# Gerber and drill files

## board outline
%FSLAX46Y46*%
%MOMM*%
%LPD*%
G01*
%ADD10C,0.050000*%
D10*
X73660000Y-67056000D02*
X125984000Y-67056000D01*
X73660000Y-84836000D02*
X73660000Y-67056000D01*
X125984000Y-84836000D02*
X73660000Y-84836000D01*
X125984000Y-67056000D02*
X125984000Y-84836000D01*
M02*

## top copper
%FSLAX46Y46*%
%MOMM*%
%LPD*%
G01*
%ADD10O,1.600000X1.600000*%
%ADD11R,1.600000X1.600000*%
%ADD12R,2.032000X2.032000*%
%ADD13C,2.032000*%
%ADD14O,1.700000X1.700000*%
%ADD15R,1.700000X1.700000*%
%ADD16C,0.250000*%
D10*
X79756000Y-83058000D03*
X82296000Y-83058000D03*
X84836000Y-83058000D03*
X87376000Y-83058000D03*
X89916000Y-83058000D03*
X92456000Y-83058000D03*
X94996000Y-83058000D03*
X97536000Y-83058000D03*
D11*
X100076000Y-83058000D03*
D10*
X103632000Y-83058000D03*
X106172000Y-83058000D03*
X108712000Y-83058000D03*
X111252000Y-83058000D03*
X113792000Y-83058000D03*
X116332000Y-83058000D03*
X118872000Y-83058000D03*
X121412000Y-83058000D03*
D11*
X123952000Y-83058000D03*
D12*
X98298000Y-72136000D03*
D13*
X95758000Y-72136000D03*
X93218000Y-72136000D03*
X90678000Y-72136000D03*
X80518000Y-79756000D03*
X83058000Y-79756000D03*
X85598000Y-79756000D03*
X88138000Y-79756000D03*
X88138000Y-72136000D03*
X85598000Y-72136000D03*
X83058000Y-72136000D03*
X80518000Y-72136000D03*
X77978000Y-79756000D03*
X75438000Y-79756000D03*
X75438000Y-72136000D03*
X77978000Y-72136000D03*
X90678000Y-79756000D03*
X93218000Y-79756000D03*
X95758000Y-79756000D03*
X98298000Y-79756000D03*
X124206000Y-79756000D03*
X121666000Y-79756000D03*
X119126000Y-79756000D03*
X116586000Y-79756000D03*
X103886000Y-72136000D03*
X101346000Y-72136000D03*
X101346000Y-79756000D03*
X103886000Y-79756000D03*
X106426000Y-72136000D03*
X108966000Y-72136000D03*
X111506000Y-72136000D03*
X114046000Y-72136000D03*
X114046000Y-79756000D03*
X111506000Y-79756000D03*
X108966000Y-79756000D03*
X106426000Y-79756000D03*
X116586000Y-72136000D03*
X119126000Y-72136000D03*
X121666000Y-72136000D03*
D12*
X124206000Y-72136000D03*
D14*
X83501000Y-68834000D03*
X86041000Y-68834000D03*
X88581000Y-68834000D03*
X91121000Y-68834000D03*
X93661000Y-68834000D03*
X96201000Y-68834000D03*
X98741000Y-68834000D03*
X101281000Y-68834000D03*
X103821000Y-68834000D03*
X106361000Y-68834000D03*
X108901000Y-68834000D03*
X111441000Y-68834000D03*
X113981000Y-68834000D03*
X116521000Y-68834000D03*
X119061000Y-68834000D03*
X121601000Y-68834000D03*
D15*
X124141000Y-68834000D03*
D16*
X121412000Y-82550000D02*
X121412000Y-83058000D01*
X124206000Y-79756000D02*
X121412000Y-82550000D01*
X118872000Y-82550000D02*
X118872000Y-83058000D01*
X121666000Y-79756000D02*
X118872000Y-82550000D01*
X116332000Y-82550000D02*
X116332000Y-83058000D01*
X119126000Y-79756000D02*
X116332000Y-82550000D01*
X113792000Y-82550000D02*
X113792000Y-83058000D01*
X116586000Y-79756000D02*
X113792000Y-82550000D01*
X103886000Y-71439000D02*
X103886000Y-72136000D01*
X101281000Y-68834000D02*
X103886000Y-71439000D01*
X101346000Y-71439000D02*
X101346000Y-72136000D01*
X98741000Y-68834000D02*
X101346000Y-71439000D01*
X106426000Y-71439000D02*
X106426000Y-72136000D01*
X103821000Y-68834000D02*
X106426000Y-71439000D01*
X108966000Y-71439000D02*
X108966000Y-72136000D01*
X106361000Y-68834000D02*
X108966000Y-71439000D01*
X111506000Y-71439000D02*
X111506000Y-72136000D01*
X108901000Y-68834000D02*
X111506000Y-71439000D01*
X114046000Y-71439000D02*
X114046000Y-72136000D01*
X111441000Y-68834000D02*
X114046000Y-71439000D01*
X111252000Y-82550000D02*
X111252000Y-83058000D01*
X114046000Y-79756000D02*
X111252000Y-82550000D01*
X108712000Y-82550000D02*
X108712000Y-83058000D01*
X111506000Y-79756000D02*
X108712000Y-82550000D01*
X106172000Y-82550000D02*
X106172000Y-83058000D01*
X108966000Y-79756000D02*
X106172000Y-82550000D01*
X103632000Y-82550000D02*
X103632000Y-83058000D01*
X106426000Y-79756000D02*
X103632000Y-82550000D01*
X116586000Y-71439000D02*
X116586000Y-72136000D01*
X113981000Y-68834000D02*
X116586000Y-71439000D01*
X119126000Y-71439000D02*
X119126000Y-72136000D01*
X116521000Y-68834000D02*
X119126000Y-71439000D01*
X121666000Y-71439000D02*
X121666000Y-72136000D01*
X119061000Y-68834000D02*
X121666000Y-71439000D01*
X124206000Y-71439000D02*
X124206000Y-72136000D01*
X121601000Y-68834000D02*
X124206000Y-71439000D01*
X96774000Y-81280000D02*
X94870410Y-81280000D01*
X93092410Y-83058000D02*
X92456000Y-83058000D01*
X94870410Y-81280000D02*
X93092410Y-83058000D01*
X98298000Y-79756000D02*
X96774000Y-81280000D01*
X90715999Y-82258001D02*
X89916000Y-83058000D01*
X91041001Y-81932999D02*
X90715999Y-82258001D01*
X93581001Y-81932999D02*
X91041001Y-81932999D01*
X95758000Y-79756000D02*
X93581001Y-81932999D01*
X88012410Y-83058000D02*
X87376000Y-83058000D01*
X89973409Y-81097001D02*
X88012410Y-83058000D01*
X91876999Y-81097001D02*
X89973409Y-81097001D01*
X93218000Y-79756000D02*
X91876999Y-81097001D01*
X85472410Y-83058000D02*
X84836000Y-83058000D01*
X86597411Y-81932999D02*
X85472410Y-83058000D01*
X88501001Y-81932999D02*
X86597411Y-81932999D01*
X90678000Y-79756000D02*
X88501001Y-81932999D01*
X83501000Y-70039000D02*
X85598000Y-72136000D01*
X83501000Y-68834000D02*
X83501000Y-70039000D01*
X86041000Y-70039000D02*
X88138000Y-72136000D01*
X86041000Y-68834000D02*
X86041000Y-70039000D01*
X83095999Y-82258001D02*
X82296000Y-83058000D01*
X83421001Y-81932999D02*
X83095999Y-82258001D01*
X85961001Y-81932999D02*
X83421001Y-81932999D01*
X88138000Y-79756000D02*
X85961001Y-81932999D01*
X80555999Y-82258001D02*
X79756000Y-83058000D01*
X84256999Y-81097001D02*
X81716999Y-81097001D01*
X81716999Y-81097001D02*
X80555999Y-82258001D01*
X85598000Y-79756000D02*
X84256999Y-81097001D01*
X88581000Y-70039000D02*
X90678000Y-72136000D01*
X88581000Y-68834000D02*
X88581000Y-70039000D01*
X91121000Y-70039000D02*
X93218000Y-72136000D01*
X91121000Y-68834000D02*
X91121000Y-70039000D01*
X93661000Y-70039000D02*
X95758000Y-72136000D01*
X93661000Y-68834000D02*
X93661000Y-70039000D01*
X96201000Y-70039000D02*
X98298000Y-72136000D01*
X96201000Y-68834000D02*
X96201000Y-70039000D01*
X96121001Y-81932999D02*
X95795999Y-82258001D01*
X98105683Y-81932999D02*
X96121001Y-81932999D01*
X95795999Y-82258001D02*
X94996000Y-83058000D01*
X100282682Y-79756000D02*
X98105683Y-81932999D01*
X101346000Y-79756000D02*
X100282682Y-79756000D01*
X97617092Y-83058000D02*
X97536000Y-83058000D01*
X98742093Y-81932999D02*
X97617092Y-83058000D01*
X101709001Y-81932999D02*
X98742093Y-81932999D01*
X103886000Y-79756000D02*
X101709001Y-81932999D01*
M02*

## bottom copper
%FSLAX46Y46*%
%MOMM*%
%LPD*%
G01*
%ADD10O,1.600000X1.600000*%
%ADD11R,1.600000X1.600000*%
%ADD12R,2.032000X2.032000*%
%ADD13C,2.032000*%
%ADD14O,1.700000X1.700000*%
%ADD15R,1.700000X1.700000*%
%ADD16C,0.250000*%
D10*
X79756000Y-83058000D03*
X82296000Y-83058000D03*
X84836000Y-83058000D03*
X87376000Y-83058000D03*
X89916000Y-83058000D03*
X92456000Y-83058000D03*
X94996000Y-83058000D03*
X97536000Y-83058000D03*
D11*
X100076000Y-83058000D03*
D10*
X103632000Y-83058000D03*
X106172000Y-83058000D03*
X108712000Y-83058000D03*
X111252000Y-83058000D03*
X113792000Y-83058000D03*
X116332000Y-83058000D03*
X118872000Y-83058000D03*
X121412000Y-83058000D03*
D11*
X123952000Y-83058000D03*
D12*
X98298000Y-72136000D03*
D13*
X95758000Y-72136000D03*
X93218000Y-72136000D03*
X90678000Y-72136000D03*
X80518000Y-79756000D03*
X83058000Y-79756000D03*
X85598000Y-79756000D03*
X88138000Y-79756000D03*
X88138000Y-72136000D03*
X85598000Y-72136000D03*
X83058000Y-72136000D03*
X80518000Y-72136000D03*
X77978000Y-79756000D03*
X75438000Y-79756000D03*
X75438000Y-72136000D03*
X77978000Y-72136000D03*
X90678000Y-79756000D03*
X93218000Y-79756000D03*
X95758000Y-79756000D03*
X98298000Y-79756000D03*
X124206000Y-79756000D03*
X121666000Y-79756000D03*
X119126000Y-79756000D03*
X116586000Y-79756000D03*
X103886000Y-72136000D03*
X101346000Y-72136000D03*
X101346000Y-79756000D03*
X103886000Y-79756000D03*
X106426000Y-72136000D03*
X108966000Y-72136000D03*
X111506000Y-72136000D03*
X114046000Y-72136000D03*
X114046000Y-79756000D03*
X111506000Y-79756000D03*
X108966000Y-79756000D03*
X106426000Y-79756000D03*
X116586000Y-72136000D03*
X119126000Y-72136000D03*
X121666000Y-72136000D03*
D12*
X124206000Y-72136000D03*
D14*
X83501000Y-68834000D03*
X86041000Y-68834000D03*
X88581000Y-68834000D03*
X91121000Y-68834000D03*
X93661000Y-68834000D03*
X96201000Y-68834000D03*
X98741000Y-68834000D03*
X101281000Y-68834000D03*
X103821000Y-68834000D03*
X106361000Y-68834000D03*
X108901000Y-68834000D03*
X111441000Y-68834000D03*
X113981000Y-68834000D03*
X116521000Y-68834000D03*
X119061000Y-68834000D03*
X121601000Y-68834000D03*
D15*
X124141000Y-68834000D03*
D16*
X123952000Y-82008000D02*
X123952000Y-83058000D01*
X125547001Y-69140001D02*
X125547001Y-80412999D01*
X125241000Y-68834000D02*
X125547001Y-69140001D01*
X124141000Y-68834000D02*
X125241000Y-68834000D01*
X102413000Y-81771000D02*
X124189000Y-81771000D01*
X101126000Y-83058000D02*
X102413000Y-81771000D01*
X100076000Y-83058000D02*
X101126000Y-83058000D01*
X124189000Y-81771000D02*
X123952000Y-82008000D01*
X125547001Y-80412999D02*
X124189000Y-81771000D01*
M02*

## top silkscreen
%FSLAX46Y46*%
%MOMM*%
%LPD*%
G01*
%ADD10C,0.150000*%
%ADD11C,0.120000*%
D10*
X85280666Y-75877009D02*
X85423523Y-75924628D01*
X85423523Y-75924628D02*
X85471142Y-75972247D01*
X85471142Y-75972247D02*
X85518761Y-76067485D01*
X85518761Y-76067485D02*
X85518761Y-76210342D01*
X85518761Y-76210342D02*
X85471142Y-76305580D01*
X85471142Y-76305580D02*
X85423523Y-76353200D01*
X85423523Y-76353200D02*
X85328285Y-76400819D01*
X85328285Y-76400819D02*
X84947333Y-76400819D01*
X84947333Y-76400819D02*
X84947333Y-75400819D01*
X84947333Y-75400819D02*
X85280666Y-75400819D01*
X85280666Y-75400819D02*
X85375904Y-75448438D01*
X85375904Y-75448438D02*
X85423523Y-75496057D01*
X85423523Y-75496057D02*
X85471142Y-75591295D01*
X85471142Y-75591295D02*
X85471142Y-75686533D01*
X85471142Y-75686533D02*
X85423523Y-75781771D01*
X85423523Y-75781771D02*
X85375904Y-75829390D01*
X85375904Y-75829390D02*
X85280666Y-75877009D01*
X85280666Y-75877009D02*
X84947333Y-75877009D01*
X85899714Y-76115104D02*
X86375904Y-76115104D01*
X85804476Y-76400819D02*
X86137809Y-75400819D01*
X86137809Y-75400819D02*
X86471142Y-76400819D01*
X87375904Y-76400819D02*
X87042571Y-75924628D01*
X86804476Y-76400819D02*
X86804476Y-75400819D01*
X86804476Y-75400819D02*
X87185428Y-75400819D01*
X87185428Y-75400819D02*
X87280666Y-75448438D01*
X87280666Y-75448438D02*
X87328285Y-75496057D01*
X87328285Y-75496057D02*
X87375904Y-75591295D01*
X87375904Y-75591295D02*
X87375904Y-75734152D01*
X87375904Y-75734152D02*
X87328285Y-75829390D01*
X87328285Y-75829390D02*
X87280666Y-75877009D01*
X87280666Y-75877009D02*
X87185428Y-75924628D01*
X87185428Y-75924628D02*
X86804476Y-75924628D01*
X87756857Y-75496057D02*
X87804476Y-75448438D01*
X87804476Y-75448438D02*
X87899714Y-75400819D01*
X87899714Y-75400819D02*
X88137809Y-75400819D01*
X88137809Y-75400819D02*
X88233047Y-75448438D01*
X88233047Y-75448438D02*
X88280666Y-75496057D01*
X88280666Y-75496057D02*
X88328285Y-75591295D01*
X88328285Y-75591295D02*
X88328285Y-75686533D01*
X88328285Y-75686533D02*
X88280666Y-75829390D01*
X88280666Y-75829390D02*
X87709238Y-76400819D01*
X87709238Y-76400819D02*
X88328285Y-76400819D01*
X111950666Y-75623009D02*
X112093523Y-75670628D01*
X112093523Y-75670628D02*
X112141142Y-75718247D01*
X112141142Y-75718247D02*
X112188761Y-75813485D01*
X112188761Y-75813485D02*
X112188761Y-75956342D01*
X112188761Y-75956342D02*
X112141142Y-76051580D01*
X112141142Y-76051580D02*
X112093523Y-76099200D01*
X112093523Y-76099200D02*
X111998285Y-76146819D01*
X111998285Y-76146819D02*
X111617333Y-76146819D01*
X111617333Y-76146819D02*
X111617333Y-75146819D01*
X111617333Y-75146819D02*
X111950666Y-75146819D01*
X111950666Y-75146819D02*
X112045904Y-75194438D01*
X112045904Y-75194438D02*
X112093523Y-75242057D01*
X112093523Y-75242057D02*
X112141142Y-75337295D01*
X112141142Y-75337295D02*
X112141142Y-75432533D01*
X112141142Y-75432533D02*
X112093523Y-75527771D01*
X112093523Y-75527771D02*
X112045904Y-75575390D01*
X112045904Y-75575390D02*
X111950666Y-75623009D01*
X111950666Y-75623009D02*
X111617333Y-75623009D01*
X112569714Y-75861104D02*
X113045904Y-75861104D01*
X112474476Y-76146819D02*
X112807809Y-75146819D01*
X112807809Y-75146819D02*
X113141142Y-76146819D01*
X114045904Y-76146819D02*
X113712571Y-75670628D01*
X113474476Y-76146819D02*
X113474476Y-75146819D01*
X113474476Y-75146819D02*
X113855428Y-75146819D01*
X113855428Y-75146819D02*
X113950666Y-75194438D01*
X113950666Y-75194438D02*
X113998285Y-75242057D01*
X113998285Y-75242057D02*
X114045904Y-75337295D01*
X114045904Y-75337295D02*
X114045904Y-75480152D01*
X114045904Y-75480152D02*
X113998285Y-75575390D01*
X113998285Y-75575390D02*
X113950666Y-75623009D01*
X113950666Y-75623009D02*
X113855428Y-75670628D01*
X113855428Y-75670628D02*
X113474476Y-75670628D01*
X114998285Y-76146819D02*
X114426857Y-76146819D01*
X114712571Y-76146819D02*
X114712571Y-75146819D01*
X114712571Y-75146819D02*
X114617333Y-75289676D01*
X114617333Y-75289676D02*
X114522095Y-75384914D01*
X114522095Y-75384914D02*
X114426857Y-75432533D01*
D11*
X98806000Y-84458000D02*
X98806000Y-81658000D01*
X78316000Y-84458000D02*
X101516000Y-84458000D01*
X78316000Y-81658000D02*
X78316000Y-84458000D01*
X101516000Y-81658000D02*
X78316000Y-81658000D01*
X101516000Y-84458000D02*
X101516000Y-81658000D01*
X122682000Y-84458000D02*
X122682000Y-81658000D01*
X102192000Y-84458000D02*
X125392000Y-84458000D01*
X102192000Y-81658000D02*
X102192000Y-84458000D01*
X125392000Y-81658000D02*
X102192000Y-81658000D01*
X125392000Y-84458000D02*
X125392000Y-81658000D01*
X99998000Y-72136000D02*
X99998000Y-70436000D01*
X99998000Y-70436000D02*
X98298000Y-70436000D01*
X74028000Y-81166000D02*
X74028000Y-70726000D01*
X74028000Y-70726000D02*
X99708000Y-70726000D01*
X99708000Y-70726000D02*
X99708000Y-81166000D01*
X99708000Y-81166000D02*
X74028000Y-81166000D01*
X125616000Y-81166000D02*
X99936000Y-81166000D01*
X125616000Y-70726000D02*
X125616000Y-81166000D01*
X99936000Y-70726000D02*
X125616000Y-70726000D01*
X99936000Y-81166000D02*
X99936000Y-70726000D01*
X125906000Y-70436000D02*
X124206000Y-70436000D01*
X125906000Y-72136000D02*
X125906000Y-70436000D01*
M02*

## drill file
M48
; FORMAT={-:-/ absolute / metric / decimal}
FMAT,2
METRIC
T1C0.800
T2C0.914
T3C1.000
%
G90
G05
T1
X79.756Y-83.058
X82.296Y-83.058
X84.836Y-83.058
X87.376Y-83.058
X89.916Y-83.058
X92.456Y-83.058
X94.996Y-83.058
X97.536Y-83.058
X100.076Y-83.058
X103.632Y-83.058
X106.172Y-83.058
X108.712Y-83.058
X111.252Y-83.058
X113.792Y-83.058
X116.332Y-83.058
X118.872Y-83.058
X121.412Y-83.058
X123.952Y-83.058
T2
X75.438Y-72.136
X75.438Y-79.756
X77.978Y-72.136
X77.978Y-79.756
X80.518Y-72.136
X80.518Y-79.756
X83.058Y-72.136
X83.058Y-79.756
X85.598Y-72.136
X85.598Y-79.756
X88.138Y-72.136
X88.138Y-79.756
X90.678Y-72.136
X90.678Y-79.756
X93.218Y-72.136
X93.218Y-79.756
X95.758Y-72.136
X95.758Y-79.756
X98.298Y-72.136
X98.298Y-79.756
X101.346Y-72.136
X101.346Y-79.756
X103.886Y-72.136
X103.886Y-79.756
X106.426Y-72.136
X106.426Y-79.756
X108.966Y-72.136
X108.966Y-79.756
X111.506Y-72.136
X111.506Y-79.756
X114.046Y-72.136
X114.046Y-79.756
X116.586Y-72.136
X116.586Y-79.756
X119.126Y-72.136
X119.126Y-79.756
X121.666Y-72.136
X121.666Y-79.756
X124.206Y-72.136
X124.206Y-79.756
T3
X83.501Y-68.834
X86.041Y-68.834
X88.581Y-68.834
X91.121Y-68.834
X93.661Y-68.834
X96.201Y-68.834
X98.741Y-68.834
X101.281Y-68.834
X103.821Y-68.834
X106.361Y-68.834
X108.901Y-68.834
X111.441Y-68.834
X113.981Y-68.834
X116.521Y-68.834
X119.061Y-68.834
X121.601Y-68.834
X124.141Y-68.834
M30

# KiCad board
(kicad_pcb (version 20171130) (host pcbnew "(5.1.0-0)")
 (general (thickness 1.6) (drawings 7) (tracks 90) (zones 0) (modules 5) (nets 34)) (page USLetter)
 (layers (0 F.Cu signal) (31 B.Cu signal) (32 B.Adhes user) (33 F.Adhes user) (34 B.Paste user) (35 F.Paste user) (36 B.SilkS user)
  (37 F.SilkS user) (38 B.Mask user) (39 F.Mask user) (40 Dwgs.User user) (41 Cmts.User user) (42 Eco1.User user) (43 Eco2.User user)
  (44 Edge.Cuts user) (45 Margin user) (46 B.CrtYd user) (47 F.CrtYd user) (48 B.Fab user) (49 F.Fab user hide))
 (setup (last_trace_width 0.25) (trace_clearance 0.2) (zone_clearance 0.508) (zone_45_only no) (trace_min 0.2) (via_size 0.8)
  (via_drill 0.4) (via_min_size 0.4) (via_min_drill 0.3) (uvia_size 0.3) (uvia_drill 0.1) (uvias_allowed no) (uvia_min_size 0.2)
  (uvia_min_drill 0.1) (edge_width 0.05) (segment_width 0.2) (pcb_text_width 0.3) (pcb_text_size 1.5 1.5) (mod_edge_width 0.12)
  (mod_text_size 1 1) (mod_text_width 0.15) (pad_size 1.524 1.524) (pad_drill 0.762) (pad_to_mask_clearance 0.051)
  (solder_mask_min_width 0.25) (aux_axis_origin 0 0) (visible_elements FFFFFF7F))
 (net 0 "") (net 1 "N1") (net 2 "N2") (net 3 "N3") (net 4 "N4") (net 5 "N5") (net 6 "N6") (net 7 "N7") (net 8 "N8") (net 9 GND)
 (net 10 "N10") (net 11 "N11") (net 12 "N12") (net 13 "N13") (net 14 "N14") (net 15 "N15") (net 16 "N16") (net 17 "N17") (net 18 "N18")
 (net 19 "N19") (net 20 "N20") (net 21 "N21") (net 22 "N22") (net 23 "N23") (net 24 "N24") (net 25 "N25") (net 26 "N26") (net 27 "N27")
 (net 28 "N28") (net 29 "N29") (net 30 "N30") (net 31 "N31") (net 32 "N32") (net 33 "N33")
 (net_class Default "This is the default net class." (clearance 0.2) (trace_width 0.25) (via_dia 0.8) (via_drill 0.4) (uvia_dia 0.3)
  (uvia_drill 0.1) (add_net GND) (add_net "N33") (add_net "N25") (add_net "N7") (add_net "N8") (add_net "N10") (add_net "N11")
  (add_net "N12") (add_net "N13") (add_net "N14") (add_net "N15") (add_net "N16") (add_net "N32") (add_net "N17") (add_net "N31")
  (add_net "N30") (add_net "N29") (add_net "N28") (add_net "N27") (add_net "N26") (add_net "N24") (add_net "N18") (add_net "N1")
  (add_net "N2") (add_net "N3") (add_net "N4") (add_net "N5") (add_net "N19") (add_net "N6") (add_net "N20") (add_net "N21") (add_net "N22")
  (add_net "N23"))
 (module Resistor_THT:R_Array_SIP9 (layer F.Cu) (at 100.076 83.058 180)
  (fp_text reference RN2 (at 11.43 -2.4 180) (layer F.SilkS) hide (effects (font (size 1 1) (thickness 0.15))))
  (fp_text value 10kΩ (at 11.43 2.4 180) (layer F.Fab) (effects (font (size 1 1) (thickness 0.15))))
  (fp_line (start 1.27 -1.4) (end 1.27 1.4) (layer F.SilkS) (width 0.12))
  (fp_line (start 21.76 -1.4) (end -1.44 -1.4) (layer F.SilkS) (width 0.12))
  (fp_line (start 21.76 1.4) (end 21.76 -1.4) (layer F.SilkS) (width 0.12))
  (fp_line (start -1.44 1.4) (end 21.76 1.4) (layer F.SilkS) (width 0.12))
  (fp_line (start -1.44 -1.4) (end -1.44 1.4) (layer F.SilkS) (width 0.12))
  (pad 9 thru_hole oval (at 20.32 0 180) (size 1.6 1.6) (drill 0.8) (layers *.Cu *.Mask) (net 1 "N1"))
  (pad 8 thru_hole oval (at 17.78 0 180) (size 1.6 1.6) (drill 0.8) (layers *.Cu *.Mask) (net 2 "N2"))
  (pad 7 thru_hole oval (at 15.24 0 180) (size 1.6 1.6) (drill 0.8) (layers *.Cu *.Mask) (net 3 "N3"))
  (pad 6 thru_hole oval (at 12.7 0 180) (size 1.6 1.6) (drill 0.8) (layers *.Cu *.Mask) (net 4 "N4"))
  (pad 5 thru_hole oval (at 10.16 0 180) (size 1.6 1.6) (drill 0.8) (layers *.Cu *.Mask) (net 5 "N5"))
  (pad 4 thru_hole oval (at 7.62 0 180) (size 1.6 1.6) (drill 0.8) (layers *.Cu *.Mask) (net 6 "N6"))
  (pad 3 thru_hole oval (at 5.08 0 180) (size 1.6 1.6) (drill 0.8) (layers *.Cu *.Mask) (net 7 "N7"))
  (pad 2 thru_hole oval (at 2.54 0 180) (size 1.6 1.6) (drill 0.8) (layers *.Cu *.Mask) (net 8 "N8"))
  (pad 1 thru_hole rect (at 0 0 180) (size 1.6 1.6) (drill 0.8) (layers *.Cu *.Mask) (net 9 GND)))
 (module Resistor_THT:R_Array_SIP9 (layer F.Cu) (at 123.952 83.058 180)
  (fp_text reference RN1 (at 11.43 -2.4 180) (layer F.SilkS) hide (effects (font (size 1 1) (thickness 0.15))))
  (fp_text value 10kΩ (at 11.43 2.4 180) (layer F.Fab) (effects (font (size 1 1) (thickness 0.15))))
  (fp_line (start 1.27 -1.4) (end 1.27 1.4) (layer F.SilkS) (width 0.12))
  (fp_line (start 21.76 -1.4) (end -1.44 -1.4) (layer F.SilkS) (width 0.12))
  (fp_line (start 21.76 1.4) (end 21.76 -1.4) (layer F.SilkS) (width 0.12))
  (fp_line (start -1.44 1.4) (end 21.76 1.4) (layer F.SilkS) (width 0.12))
  (fp_line (start -1.44 -1.4) (end -1.44 1.4) (layer F.SilkS) (width 0.12))
  (pad 9 thru_hole oval (at 20.32 0 180) (size 1.6 1.6) (drill 0.8) (layers *.Cu *.Mask) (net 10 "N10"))
  (pad 8 thru_hole oval (at 17.78 0 180) (size 1.6 1.6) (drill 0.8) (layers *.Cu *.Mask) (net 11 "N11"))
  (pad 7 thru_hole oval (at 15.24 0 180) (size 1.6 1.6) (drill 0.8) (layers *.Cu *.Mask) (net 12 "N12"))
  (pad 6 thru_hole oval (at 12.7 0 180) (size 1.6 1.6) (drill 0.8) (layers *.Cu *.Mask) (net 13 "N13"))
  (pad 5 thru_hole oval (at 10.16 0 180) (size 1.6 1.6) (drill 0.8) (layers *.Cu *.Mask) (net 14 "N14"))
  (pad 4 thru_hole oval (at 7.62 0 180) (size 1.6 1.6) (drill 0.8) (layers *.Cu *.Mask) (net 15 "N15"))
  (pad 3 thru_hole oval (at 5.08 0 180) (size 1.6 1.6) (drill 0.8) (layers *.Cu *.Mask) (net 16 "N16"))
  (pad 2 thru_hole oval (at 2.54 0 180) (size 1.6 1.6) (drill 0.8) (layers *.Cu *.Mask) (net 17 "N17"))
  (pad 1 thru_hole rect (at 0 0 180) (size 1.6 1.6) (drill 0.8) (layers *.Cu *.Mask) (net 9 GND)))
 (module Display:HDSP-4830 (layer F.Cu) (at 98.298 72.136 270)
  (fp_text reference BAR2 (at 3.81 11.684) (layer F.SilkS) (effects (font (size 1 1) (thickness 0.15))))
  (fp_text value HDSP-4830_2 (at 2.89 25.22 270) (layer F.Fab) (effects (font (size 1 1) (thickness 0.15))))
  (fp_line (start 0 -1.7) (end -1.7 -1.7) (layer F.SilkS) (width 0.12))
  (fp_line (start -1.7 -1.7) (end -1.7 0) (layer F.SilkS) (width 0.12))
  (fp_line (start 9.03 24.27) (end -1.41 24.27) (layer F.SilkS) (width 0.12))
  (fp_line (start -1.41 24.27) (end -1.41 -1.41) (layer F.SilkS) (width 0.12))
  (fp_line (start -1.41 -1.41) (end 9.03 -1.41) (layer F.SilkS) (width 0.12))
  (fp_line (start 9.03 -1.41) (end 9.03 24.27) (layer F.SilkS) (width 0.12))
  (pad 1 thru_hole rect (at 0 0 180) (size 2.032 2.032) (drill 0.9144) (layers *.Cu *.Mask) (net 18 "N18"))
  (pad 2 thru_hole circle (at 0 2.54 180) (size 2.032 2.032) (drill 0.9144) (layers *.Cu *.Mask) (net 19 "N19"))
  (pad 3 thru_hole circle (at 0 5.08 180) (size 2.032 2.032) (drill 0.9144) (layers *.Cu *.Mask) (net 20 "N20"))
  (pad 4 thru_hole circle (at 0 7.62 180) (size 2.032 2.032) (drill 0.9144) (layers *.Cu *.Mask) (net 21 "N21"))
  (pad 13 thru_hole circle (at 7.62 17.78 180) (size 2.032 2.032) (drill 0.9144) (layers *.Cu *.Mask))
  (pad 14 thru_hole circle (at 7.62 15.24 180) (size 2.032 2.032) (drill 0.9144) (layers *.Cu *.Mask))
  (pad 15 thru_hole circle (at 7.62 12.7 180) (size 2.032 2.032) (drill 0.9144) (layers *.Cu *.Mask) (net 1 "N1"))
  (pad 16 thru_hole circle (at 7.62 10.16 180) (size 2.032 2.032) (drill 0.9144) (layers *.Cu *.Mask) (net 2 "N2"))
  (pad 5 thru_hole circle (at 0 10.16 180) (size 2.032 2.032) (drill 0.9144) (layers *.Cu *.Mask) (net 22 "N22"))
  (pad 6 thru_hole circle (at 0 12.7 180) (size 2.032 2.032) (drill 0.9144) (layers *.Cu *.Mask) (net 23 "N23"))
  (pad 7 thru_hole circle (at 0 15.24 180) (size 2.032 2.032) (drill 0.9144) (layers *.Cu *.Mask))
  (pad 8 thru_hole circle (at 0 17.78 180) (size 2.032 2.032) (drill 0.9144) (layers *.Cu *.Mask))
  (pad 12 thru_hole circle (at 7.62 20.32 180) (size 2.032 2.032) (drill 0.9144) (layers *.Cu *.Mask))
  (pad 11 thru_hole circle (at 7.62 22.86 180) (size 2.032 2.032) (drill 0.9144) (layers *.Cu *.Mask))
  (pad 10 thru_hole circle (at 0 22.86 180) (size 2.032 2.032) (drill 0.9144) (layers *.Cu *.Mask))
  (pad 9 thru_hole circle (at 0 20.32 180) (size 2.032 2.032) (drill 0.9144) (layers *.Cu *.Mask))
  (pad 17 thru_hole circle (at 7.62 7.62 180) (size 2.032 2.032) (drill 0.9144) (layers *.Cu *.Mask) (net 3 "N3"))
  (pad 18 thru_hole circle (at 7.62 5.08 180) (size 2.032 2.032) (drill 0.9144) (layers *.Cu *.Mask) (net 4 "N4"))
  (pad 19 thru_hole circle (at 7.62 2.54 180) (size 2.032 2.032) (drill 0.9144) (layers *.Cu *.Mask) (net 5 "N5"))
  (pad 20 thru_hole circle (at 7.62 0 180) (size 2.032 2.032) (drill 0.9144) (layers *.Cu *.Mask) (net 6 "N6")))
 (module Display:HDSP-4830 (layer F.Cu) (at 124.206 72.136 270)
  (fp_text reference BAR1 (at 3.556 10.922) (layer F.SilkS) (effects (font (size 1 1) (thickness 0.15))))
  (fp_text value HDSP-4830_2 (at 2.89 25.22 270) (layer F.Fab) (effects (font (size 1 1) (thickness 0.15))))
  (fp_line (start 9.03 -1.41) (end 9.03 24.27) (layer F.SilkS) (width 0.12))
  (fp_line (start -1.41 -1.41) (end 9.03 -1.41) (layer F.SilkS) (width 0.12))
  (fp_line (start -1.41 24.27) (end -1.41 -1.41) (layer F.SilkS) (width 0.12))
  (fp_line (start 9.03 24.27) (end -1.41 24.27) (layer F.SilkS) (width 0.12))
  (fp_line (start -1.7 -1.7) (end -1.7 0) (layer F.SilkS) (width 0.12))
  (fp_line (start 0 -1.7) (end -1.7 -1.7) (layer F.SilkS) (width 0.12))
  (pad 20 thru_hole circle (at 7.62 0 180) (size 2.032 2.032) (drill 0.9144) (layers *.Cu *.Mask) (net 17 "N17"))
  (pad 19 thru_hole circle (at 7.62 2.54 180) (size 2.032 2.032) (drill 0.9144) (layers *.Cu *.Mask) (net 16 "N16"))
  (pad 18 thru_hole circle (at 7.62 5.08 180) (size 2.032 2.032) (drill 0.9144) (layers *.Cu *.Mask) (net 15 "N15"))
  (pad 17 thru_hole circle (at 7.62 7.62 180) (size 2.032 2.032) (drill 0.9144) (layers *.Cu *.Mask) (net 14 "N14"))
  (pad 9 thru_hole circle (at 0 20.32 180) (size 2.032 2.032) (drill 0.9144) (layers *.Cu *.Mask) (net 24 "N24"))
  (pad 10 thru_hole circle (at 0 22.86 180) (size 2.032 2.032) (drill 0.9144) (layers *.Cu *.Mask) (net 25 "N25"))
  (pad 11 thru_hole circle (at 7.62 22.86 180) (size 2.032 2.032) (drill 0.9144) (layers *.Cu *.Mask) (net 7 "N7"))
  (pad 12 thru_hole circle (at 7.62 20.32 180) (size 2.032 2.032) (drill 0.9144) (layers *.Cu *.Mask) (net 8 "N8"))
  (pad 8 thru_hole circle (at 0 17.78 180) (size 2.032 2.032) (drill 0.9144) (layers *.Cu *.Mask) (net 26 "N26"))
  (pad 7 thru_hole circle (at 0 15.24 180) (size 2.032 2.032) (drill 0.9144) (layers *.Cu *.Mask) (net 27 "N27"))
  (pad 6 thru_hole circle (at 0 12.7 180) (size 2.032 2.032) (drill 0.9144) (layers *.Cu *.Mask) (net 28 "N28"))
  (pad 5 thru_hole circle (at 0 10.16 180) (size 2.032 2.032) (drill 0.9144) (layers *.Cu *.Mask) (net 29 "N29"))
  (pad 16 thru_hole circle (at 7.62 10.16 180) (size 2.032 2.032) (drill 0.9144) (layers *.Cu *.Mask) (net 13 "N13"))
  (pad 15 thru_hole circle (at 7.62 12.7 180) (size 2.032 2.032) (drill 0.9144) (layers *.Cu *.Mask) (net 12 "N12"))
  (pad 14 thru_hole circle (at 7.62 15.24 180) (size 2.032 2.032) (drill 0.9144) (layers *.Cu *.Mask) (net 11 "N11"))
  (pad 13 thru_hole circle (at 7.62 17.78 180) (size 2.032 2.032) (drill 0.9144) (layers *.Cu *.Mask) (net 10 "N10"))
  (pad 4 thru_hole circle (at 0 7.62 180) (size 2.032 2.032) (drill 0.9144) (layers *.Cu *.Mask) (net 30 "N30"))
  (pad 3 thru_hole circle (at 0 5.08 180) (size 2.032 2.032) (drill 0.9144) (layers *.Cu *.Mask) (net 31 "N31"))
  (pad 2 thru_hole circle (at 0 2.54 180) (size 2.032 2.032) (drill 0.9144) (layers *.Cu *.Mask) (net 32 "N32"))
  (pad 1 thru_hole rect (at 0 0 180) (size 2.032 2.032) (drill 0.9144) (layers *.Cu *.Mask) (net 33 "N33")))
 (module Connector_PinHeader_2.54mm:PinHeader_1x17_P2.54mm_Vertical (layer B.Cu) (at 124.141 68.834 90)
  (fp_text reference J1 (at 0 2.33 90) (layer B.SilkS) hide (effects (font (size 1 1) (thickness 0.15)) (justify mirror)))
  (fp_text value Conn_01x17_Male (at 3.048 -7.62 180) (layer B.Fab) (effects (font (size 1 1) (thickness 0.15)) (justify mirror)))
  (pad 17 thru_hole oval (at 0 -40.64 90) (size 1.7 1.7) (drill 1) (layers *.Cu *.Mask) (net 23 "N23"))
  (pad 16 thru_hole oval (at 0 -38.1 90) (size 1.7 1.7) (drill 1) (layers *.Cu *.Mask) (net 22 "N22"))
  (pad 15 thru_hole oval (at 0 -35.56 90) (size 1.7 1.7) (drill 1) (layers *.Cu *.Mask) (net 21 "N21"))
  (pad 14 thru_hole oval (at 0 -33.02 90) (size 1.7 1.7) (drill 1) (layers *.Cu *.Mask) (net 20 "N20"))
  (pad 13 thru_hole oval (at 0 -30.48 90) (size 1.7 1.7) (drill 1) (layers *.Cu *.Mask) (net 19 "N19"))
  (pad 12 thru_hole oval (at 0 -27.94 90) (size 1.7 1.7) (drill 1) (layers *.Cu *.Mask) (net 18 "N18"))
  (pad 11 thru_hole oval (at 0 -25.4 90) (size 1.7 1.7) (drill 1) (layers *.Cu *.Mask) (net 25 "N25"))
  (pad 10 thru_hole oval (at 0 -22.86 90) (size 1.7 1.7) (drill 1) (layers *.Cu *.Mask) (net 24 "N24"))
  (pad 9 thru_hole oval (at 0 -20.32 90) (size 1.7 1.7) (drill 1) (layers *.Cu *.Mask) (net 26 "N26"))
  (pad 8 thru_hole oval (at 0 -17.78 90) (size 1.7 1.7) (drill 1) (layers *.Cu *.Mask) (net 27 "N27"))
  (pad 7 thru_hole oval (at 0 -15.24 90) (size 1.7 1.7) (drill 1) (layers *.Cu *.Mask) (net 28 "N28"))
  (pad 6 thru_hole oval (at 0 -12.7 90) (size 1.7 1.7) (drill 1) (layers *.Cu *.Mask) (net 29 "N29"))
  (pad 5 thru_hole oval (at 0 -10.16 90) (size 1.7 1.7) (drill 1) (layers *.Cu *.Mask) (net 30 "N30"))
  (pad 4 thru_hole oval (at 0 -7.62 90) (size 1.7 1.7) (drill 1) (layers *.Cu *.Mask) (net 31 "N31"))
  (pad 3 thru_hole oval (at 0 -5.08 90) (size 1.7 1.7) (drill 1) (layers *.Cu *.Mask) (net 32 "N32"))
  (pad 2 thru_hole oval (at 0 -2.54 90) (size 1.7 1.7) (drill 1) (layers *.Cu *.Mask) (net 33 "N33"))
  (pad 1 thru_hole rect (at 0 0 90) (size 1.7 1.7) (drill 1) (layers *.Cu *.Mask) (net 9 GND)))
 (gr_line (start 73.66 67.056) (end 125.984 67.056) (layer Edge.Cuts) (width 0.05))
 (gr_line (start 73.66 84.836) (end 73.66 67.056) (layer Edge.Cuts) (width 0.05))
 (gr_line (start 125.984 84.836) (end 73.66 84.836) (layer Edge.Cuts) (width 0.05))
 (gr_line (start 125.984 67.056) (end 125.984 84.836) (layer Edge.Cuts) (width 0.05))
 (segment (start 123.952 82.008) (end 123.952 83.058) (width 0.25) (layer B.Cu) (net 9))
 (segment (start 125.547001 69.140001) (end 125.547001 80.412999) (width 0.25) (layer B.Cu) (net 9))
 (segment (start 125.241 68.834) (end 125.547001 69.140001) (width 0.25) (layer B.Cu) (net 9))
 (segment (start 124.141 68.834) (end 125.241 68.834) (width 0.25) (layer B.Cu) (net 9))
 (segment (start 102.413 81.771) (end 124.189 81.771) (width 0.25) (layer B.Cu) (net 9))
 (segment (start 101.126 83.058) (end 102.413 81.771) (width 0.25) (layer B.Cu) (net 9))
 (segment (start 100.076 83.058) (end 101.126 83.058) (width 0.25) (layer B.Cu) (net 9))
 (segment (start 124.189 81.771) (end 123.952 82.008) (width 0.25) (layer B.Cu) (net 9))
 (segment (start 125.547001 80.412999) (end 124.189 81.771) (width 0.25) (layer B.Cu) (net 9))
 (segment (start 121.412 82.55) (end 121.412 83.058) (width 0.25) (layer F.Cu) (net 17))
 (segment (start 124.206 79.756) (end 121.412 82.55) (width 0.25) (layer F.Cu) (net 17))
 (segment (start 118.872 82.55) (end 118.872 83.058) (width 0.25) (layer F.Cu) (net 16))
 (segment (start 121.666 79.756) (end 118.872 82.55) (width 0.25) (layer F.Cu) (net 16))
 (segment (start 116.332 82.55) (end 116.332 83.058) (width 0.25) (layer F.Cu) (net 15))
 (segment (start 119.126 79.756) (end 116.332 82.55) (width 0.25) (layer F.Cu) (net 15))
 (segment (start 113.792 82.55) (end 113.792 83.058) (width 0.25) (layer F.Cu) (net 14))
 (segment (start 116.586 79.756) (end 113.792 82.55) (width 0.25) (layer F.Cu) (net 14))
 (segment (start 103.886 71.439) (end 103.886 72.136) (width 0.25) (layer F.Cu) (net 24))
 (segment (start 101.281 68.834) (end 103.886 71.439) (width 0.25) (layer F.Cu) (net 24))
 (segment (start 101.346 71.439) (end 101.346 72.136) (width 0.25) (layer F.Cu) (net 25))
 (segment (start 98.741 68.834) (end 101.346 71.439) (width 0.25) (layer F.Cu) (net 25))
 (segment (start 106.426 71.439) (end 106.426 72.136) (width 0.25) (layer F.Cu) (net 26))
 (segment (start 103.821 68.834) (end 106.426 71.439) (width 0.25) (layer F.Cu) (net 26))
 (segment (start 108.966 71.439) (end 108.966 72.136) (width 0.25) (layer F.Cu) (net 27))
 (segment (start 106.361 68.834) (end 108.966 71.439) (width 0.25) (layer F.Cu) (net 27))
 (segment (start 111.506 71.439) (end 111.506 72.136) (width 0.25) (layer F.Cu) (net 28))
 (segment (start 108.901 68.834) (end 111.506 71.439) (width 0.25) (layer F.Cu) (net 28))
 (segment (start 114.046 71.439) (end 114.046 72.136) (width 0.25) (layer F.Cu) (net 29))
 (segment (start 111.441 68.834) (end 114.046 71.439) (width 0.25) (layer F.Cu) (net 29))
 (segment (start 111.252 82.55) (end 111.252 83.058) (width 0.25) (layer F.Cu) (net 13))
 (segment (start 114.046 79.756) (end 111.252 82.55) (width 0.25) (layer F.Cu) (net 13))
 (segment (start 108.712 82.55) (end 108.712 83.058) (width 0.25) (layer F.Cu) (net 12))
 (segment (start 111.506 79.756) (end 108.712 82.55) (width 0.25) (layer F.Cu) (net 12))
 (segment (start 106.172 82.55) (end 106.172 83.058) (width 0.25) (layer F.Cu) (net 11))
 (segment (start 108.966 79.756) (end 106.172 82.55) (width 0.25) (layer F.Cu) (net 11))
 (segment (start 103.632 82.55) (end 103.632 83.058) (width 0.25) (layer F.Cu) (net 10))
 (segment (start 106.426 79.756) (end 103.632 82.55) (width 0.25) (layer F.Cu) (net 10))
 (segment (start 116.586 71.439) (end 116.586 72.136) (width 0.25) (layer F.Cu) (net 30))
 (segment (start 113.981 68.834) (end 116.586 71.439) (width 0.25) (layer F.Cu) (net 30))
 (segment (start 119.126 71.439) (end 119.126 72.136) (width 0.25) (layer F.Cu) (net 31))
 (segment (start 116.521 68.834) (end 119.126 71.439) (width 0.25) (layer F.Cu) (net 31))
 (segment (start 121.666 71.439) (end 121.666 72.136) (width 0.25) (layer F.Cu) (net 32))
 (segment (start 119.061 68.834) (end 121.666 71.439) (width 0.25) (layer F.Cu) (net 32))
 (segment (start 124.206 71.439) (end 124.206 72.136) (width 0.25) (layer F.Cu) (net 33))
 (segment (start 121.601 68.834) (end 124.206 71.439) (width 0.25) (layer F.Cu) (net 33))
 (segment (start 96.774 81.28) (end 94.87041 81.28) (width 0.25) (layer F.Cu) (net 6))
 (segment (start 93.09241 83.058) (end 92.456 83.058) (width 0.25) (layer F.Cu) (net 6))
 (segment (start 94.87041 81.28) (end 93.09241 83.058) (width 0.25) (layer F.Cu) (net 6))
 (segment (start 98.298 79.756) (end 96.774 81.28) (width 0.25) (layer F.Cu) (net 6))
 (segment (start 90.715999 82.258001) (end 89.916 83.058) (width 0.25) (layer F.Cu) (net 5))
 (segment (start 91.041001 81.932999) (end 90.715999 82.258001) (width 0.25) (layer F.Cu) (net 5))
 (segment (start 93.581001 81.932999) (end 91.041001 81.932999) (width 0.25) (layer F.Cu) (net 5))
 (segment (start 95.758 79.756) (end 93.581001 81.932999) (width 0.25) (layer F.Cu) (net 5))
 (segment (start 88.01241 83.058) (end 87.376 83.058) (width 0.25) (layer F.Cu) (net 4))
 (segment (start 89.973409 81.097001) (end 88.01241 83.058) (width 0.25) (layer F.Cu) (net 4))
 (segment (start 91.876999 81.097001) (end 89.973409 81.097001) (width 0.25) (layer F.Cu) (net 4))
 (segment (start 93.218 79.756) (end 91.876999 81.097001) (width 0.25) (layer F.Cu) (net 4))
 (segment (start 85.47241 83.058) (end 84.836 83.058) (width 0.25) (layer F.Cu) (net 3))
 (segment (start 86.597411 81.932999) (end 85.47241 83.058) (width 0.25) (layer F.Cu) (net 3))
 (segment (start 88.501001 81.932999) (end 86.597411 81.932999) (width 0.25) (layer F.Cu) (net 3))
 (segment (start 90.678 79.756) (end 88.501001 81.932999) (width 0.25) (layer F.Cu) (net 3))
 (segment (start 83.501 70.039) (end 85.598 72.136) (width 0.25) (layer F.Cu) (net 23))
 (segment (start 83.501 68.834) (end 83.501 70.039) (width 0.25) (layer F.Cu) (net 23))
 (segment (start 86.041 70.039) (end 88.138 72.136) (width 0.25) (layer F.Cu) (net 22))
 (segment (start 86.041 68.834) (end 86.041 70.039) (width 0.25) (layer F.Cu) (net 22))
 (segment (start 83.095999 82.258001) (end 82.296 83.058) (width 0.25) (layer F.Cu) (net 2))
 (segment (start 83.421001 81.932999) (end 83.095999 82.258001) (width 0.25) (layer F.Cu) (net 2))
 (segment (start 85.961001 81.932999) (end 83.421001 81.932999) (width 0.25) (layer F.Cu) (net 2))
 (segment (start 88.138 79.756) (end 85.961001 81.932999) (width 0.25) (layer F.Cu) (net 2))
 (segment (start 80.555999 82.258001) (end 79.756 83.058) (width 0.25) (layer F.Cu) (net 1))
 (segment (start 84.256999 81.097001) (end 81.716999 81.097001) (width 0.25) (layer F.Cu) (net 1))
 (segment (start 81.716999 81.097001) (end 80.555999 82.258001) (width 0.25) (layer F.Cu) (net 1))
 (segment (start 85.598 79.756) (end 84.256999 81.097001) (width 0.25) (layer F.Cu) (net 1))
 (segment (start 88.581 70.039) (end 90.678 72.136) (width 0.25) (layer F.Cu) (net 21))
 (segment (start 88.581 68.834) (end 88.581 70.039) (width 0.25) (layer F.Cu) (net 21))
 (segment (start 91.121 70.039) (end 93.218 72.136) (width 0.25) (layer F.Cu) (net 20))
 (segment (start 91.121 68.834) (end 91.121 70.039) (width 0.25) (layer F.Cu) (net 20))
 (segment (start 93.661 70.039) (end 95.758 72.136) (width 0.25) (layer F.Cu) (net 19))
 (segment (start 93.661 68.834) (end 93.661 70.039) (width 0.25) (layer F.Cu) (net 19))
 (segment (start 96.201 70.039) (end 98.298 72.136) (width 0.25) (layer F.Cu) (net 18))
 (segment (start 96.201 68.834) (end 96.201 70.039) (width 0.25) (layer F.Cu) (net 18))
 (segment (start 96.121001 81.932999) (end 95.795999 82.258001) (width 0.25) (layer F.Cu) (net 7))
 (segment (start 98.105683 81.932999) (end 96.121001 81.932999) (width 0.25) (layer F.Cu) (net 7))
 (segment (start 95.795999 82.258001) (end 94.996 83.058) (width 0.25) (layer F.Cu) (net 7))
 (segment (start 100.282682 79.756) (end 98.105683 81.932999) (width 0.25) (layer F.Cu) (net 7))
 (segment (start 101.346 79.756) (end 100.282682 79.756) (width 0.25) (layer F.Cu) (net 7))
 (segment (start 97.617092 83.058) (end 97.536 83.058) (width 0.25) (layer F.Cu) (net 8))
 (segment (start 98.742093 81.932999) (end 97.617092 83.058) (width 0.25) (layer F.Cu) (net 8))
 (segment (start 101.709001 81.932999) (end 98.742093 81.932999) (width 0.25) (layer F.Cu) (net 8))
 (segment (start 103.886 79.756) (end 101.709001 81.932999) (width 0.25) (layer F.Cu) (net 8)))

